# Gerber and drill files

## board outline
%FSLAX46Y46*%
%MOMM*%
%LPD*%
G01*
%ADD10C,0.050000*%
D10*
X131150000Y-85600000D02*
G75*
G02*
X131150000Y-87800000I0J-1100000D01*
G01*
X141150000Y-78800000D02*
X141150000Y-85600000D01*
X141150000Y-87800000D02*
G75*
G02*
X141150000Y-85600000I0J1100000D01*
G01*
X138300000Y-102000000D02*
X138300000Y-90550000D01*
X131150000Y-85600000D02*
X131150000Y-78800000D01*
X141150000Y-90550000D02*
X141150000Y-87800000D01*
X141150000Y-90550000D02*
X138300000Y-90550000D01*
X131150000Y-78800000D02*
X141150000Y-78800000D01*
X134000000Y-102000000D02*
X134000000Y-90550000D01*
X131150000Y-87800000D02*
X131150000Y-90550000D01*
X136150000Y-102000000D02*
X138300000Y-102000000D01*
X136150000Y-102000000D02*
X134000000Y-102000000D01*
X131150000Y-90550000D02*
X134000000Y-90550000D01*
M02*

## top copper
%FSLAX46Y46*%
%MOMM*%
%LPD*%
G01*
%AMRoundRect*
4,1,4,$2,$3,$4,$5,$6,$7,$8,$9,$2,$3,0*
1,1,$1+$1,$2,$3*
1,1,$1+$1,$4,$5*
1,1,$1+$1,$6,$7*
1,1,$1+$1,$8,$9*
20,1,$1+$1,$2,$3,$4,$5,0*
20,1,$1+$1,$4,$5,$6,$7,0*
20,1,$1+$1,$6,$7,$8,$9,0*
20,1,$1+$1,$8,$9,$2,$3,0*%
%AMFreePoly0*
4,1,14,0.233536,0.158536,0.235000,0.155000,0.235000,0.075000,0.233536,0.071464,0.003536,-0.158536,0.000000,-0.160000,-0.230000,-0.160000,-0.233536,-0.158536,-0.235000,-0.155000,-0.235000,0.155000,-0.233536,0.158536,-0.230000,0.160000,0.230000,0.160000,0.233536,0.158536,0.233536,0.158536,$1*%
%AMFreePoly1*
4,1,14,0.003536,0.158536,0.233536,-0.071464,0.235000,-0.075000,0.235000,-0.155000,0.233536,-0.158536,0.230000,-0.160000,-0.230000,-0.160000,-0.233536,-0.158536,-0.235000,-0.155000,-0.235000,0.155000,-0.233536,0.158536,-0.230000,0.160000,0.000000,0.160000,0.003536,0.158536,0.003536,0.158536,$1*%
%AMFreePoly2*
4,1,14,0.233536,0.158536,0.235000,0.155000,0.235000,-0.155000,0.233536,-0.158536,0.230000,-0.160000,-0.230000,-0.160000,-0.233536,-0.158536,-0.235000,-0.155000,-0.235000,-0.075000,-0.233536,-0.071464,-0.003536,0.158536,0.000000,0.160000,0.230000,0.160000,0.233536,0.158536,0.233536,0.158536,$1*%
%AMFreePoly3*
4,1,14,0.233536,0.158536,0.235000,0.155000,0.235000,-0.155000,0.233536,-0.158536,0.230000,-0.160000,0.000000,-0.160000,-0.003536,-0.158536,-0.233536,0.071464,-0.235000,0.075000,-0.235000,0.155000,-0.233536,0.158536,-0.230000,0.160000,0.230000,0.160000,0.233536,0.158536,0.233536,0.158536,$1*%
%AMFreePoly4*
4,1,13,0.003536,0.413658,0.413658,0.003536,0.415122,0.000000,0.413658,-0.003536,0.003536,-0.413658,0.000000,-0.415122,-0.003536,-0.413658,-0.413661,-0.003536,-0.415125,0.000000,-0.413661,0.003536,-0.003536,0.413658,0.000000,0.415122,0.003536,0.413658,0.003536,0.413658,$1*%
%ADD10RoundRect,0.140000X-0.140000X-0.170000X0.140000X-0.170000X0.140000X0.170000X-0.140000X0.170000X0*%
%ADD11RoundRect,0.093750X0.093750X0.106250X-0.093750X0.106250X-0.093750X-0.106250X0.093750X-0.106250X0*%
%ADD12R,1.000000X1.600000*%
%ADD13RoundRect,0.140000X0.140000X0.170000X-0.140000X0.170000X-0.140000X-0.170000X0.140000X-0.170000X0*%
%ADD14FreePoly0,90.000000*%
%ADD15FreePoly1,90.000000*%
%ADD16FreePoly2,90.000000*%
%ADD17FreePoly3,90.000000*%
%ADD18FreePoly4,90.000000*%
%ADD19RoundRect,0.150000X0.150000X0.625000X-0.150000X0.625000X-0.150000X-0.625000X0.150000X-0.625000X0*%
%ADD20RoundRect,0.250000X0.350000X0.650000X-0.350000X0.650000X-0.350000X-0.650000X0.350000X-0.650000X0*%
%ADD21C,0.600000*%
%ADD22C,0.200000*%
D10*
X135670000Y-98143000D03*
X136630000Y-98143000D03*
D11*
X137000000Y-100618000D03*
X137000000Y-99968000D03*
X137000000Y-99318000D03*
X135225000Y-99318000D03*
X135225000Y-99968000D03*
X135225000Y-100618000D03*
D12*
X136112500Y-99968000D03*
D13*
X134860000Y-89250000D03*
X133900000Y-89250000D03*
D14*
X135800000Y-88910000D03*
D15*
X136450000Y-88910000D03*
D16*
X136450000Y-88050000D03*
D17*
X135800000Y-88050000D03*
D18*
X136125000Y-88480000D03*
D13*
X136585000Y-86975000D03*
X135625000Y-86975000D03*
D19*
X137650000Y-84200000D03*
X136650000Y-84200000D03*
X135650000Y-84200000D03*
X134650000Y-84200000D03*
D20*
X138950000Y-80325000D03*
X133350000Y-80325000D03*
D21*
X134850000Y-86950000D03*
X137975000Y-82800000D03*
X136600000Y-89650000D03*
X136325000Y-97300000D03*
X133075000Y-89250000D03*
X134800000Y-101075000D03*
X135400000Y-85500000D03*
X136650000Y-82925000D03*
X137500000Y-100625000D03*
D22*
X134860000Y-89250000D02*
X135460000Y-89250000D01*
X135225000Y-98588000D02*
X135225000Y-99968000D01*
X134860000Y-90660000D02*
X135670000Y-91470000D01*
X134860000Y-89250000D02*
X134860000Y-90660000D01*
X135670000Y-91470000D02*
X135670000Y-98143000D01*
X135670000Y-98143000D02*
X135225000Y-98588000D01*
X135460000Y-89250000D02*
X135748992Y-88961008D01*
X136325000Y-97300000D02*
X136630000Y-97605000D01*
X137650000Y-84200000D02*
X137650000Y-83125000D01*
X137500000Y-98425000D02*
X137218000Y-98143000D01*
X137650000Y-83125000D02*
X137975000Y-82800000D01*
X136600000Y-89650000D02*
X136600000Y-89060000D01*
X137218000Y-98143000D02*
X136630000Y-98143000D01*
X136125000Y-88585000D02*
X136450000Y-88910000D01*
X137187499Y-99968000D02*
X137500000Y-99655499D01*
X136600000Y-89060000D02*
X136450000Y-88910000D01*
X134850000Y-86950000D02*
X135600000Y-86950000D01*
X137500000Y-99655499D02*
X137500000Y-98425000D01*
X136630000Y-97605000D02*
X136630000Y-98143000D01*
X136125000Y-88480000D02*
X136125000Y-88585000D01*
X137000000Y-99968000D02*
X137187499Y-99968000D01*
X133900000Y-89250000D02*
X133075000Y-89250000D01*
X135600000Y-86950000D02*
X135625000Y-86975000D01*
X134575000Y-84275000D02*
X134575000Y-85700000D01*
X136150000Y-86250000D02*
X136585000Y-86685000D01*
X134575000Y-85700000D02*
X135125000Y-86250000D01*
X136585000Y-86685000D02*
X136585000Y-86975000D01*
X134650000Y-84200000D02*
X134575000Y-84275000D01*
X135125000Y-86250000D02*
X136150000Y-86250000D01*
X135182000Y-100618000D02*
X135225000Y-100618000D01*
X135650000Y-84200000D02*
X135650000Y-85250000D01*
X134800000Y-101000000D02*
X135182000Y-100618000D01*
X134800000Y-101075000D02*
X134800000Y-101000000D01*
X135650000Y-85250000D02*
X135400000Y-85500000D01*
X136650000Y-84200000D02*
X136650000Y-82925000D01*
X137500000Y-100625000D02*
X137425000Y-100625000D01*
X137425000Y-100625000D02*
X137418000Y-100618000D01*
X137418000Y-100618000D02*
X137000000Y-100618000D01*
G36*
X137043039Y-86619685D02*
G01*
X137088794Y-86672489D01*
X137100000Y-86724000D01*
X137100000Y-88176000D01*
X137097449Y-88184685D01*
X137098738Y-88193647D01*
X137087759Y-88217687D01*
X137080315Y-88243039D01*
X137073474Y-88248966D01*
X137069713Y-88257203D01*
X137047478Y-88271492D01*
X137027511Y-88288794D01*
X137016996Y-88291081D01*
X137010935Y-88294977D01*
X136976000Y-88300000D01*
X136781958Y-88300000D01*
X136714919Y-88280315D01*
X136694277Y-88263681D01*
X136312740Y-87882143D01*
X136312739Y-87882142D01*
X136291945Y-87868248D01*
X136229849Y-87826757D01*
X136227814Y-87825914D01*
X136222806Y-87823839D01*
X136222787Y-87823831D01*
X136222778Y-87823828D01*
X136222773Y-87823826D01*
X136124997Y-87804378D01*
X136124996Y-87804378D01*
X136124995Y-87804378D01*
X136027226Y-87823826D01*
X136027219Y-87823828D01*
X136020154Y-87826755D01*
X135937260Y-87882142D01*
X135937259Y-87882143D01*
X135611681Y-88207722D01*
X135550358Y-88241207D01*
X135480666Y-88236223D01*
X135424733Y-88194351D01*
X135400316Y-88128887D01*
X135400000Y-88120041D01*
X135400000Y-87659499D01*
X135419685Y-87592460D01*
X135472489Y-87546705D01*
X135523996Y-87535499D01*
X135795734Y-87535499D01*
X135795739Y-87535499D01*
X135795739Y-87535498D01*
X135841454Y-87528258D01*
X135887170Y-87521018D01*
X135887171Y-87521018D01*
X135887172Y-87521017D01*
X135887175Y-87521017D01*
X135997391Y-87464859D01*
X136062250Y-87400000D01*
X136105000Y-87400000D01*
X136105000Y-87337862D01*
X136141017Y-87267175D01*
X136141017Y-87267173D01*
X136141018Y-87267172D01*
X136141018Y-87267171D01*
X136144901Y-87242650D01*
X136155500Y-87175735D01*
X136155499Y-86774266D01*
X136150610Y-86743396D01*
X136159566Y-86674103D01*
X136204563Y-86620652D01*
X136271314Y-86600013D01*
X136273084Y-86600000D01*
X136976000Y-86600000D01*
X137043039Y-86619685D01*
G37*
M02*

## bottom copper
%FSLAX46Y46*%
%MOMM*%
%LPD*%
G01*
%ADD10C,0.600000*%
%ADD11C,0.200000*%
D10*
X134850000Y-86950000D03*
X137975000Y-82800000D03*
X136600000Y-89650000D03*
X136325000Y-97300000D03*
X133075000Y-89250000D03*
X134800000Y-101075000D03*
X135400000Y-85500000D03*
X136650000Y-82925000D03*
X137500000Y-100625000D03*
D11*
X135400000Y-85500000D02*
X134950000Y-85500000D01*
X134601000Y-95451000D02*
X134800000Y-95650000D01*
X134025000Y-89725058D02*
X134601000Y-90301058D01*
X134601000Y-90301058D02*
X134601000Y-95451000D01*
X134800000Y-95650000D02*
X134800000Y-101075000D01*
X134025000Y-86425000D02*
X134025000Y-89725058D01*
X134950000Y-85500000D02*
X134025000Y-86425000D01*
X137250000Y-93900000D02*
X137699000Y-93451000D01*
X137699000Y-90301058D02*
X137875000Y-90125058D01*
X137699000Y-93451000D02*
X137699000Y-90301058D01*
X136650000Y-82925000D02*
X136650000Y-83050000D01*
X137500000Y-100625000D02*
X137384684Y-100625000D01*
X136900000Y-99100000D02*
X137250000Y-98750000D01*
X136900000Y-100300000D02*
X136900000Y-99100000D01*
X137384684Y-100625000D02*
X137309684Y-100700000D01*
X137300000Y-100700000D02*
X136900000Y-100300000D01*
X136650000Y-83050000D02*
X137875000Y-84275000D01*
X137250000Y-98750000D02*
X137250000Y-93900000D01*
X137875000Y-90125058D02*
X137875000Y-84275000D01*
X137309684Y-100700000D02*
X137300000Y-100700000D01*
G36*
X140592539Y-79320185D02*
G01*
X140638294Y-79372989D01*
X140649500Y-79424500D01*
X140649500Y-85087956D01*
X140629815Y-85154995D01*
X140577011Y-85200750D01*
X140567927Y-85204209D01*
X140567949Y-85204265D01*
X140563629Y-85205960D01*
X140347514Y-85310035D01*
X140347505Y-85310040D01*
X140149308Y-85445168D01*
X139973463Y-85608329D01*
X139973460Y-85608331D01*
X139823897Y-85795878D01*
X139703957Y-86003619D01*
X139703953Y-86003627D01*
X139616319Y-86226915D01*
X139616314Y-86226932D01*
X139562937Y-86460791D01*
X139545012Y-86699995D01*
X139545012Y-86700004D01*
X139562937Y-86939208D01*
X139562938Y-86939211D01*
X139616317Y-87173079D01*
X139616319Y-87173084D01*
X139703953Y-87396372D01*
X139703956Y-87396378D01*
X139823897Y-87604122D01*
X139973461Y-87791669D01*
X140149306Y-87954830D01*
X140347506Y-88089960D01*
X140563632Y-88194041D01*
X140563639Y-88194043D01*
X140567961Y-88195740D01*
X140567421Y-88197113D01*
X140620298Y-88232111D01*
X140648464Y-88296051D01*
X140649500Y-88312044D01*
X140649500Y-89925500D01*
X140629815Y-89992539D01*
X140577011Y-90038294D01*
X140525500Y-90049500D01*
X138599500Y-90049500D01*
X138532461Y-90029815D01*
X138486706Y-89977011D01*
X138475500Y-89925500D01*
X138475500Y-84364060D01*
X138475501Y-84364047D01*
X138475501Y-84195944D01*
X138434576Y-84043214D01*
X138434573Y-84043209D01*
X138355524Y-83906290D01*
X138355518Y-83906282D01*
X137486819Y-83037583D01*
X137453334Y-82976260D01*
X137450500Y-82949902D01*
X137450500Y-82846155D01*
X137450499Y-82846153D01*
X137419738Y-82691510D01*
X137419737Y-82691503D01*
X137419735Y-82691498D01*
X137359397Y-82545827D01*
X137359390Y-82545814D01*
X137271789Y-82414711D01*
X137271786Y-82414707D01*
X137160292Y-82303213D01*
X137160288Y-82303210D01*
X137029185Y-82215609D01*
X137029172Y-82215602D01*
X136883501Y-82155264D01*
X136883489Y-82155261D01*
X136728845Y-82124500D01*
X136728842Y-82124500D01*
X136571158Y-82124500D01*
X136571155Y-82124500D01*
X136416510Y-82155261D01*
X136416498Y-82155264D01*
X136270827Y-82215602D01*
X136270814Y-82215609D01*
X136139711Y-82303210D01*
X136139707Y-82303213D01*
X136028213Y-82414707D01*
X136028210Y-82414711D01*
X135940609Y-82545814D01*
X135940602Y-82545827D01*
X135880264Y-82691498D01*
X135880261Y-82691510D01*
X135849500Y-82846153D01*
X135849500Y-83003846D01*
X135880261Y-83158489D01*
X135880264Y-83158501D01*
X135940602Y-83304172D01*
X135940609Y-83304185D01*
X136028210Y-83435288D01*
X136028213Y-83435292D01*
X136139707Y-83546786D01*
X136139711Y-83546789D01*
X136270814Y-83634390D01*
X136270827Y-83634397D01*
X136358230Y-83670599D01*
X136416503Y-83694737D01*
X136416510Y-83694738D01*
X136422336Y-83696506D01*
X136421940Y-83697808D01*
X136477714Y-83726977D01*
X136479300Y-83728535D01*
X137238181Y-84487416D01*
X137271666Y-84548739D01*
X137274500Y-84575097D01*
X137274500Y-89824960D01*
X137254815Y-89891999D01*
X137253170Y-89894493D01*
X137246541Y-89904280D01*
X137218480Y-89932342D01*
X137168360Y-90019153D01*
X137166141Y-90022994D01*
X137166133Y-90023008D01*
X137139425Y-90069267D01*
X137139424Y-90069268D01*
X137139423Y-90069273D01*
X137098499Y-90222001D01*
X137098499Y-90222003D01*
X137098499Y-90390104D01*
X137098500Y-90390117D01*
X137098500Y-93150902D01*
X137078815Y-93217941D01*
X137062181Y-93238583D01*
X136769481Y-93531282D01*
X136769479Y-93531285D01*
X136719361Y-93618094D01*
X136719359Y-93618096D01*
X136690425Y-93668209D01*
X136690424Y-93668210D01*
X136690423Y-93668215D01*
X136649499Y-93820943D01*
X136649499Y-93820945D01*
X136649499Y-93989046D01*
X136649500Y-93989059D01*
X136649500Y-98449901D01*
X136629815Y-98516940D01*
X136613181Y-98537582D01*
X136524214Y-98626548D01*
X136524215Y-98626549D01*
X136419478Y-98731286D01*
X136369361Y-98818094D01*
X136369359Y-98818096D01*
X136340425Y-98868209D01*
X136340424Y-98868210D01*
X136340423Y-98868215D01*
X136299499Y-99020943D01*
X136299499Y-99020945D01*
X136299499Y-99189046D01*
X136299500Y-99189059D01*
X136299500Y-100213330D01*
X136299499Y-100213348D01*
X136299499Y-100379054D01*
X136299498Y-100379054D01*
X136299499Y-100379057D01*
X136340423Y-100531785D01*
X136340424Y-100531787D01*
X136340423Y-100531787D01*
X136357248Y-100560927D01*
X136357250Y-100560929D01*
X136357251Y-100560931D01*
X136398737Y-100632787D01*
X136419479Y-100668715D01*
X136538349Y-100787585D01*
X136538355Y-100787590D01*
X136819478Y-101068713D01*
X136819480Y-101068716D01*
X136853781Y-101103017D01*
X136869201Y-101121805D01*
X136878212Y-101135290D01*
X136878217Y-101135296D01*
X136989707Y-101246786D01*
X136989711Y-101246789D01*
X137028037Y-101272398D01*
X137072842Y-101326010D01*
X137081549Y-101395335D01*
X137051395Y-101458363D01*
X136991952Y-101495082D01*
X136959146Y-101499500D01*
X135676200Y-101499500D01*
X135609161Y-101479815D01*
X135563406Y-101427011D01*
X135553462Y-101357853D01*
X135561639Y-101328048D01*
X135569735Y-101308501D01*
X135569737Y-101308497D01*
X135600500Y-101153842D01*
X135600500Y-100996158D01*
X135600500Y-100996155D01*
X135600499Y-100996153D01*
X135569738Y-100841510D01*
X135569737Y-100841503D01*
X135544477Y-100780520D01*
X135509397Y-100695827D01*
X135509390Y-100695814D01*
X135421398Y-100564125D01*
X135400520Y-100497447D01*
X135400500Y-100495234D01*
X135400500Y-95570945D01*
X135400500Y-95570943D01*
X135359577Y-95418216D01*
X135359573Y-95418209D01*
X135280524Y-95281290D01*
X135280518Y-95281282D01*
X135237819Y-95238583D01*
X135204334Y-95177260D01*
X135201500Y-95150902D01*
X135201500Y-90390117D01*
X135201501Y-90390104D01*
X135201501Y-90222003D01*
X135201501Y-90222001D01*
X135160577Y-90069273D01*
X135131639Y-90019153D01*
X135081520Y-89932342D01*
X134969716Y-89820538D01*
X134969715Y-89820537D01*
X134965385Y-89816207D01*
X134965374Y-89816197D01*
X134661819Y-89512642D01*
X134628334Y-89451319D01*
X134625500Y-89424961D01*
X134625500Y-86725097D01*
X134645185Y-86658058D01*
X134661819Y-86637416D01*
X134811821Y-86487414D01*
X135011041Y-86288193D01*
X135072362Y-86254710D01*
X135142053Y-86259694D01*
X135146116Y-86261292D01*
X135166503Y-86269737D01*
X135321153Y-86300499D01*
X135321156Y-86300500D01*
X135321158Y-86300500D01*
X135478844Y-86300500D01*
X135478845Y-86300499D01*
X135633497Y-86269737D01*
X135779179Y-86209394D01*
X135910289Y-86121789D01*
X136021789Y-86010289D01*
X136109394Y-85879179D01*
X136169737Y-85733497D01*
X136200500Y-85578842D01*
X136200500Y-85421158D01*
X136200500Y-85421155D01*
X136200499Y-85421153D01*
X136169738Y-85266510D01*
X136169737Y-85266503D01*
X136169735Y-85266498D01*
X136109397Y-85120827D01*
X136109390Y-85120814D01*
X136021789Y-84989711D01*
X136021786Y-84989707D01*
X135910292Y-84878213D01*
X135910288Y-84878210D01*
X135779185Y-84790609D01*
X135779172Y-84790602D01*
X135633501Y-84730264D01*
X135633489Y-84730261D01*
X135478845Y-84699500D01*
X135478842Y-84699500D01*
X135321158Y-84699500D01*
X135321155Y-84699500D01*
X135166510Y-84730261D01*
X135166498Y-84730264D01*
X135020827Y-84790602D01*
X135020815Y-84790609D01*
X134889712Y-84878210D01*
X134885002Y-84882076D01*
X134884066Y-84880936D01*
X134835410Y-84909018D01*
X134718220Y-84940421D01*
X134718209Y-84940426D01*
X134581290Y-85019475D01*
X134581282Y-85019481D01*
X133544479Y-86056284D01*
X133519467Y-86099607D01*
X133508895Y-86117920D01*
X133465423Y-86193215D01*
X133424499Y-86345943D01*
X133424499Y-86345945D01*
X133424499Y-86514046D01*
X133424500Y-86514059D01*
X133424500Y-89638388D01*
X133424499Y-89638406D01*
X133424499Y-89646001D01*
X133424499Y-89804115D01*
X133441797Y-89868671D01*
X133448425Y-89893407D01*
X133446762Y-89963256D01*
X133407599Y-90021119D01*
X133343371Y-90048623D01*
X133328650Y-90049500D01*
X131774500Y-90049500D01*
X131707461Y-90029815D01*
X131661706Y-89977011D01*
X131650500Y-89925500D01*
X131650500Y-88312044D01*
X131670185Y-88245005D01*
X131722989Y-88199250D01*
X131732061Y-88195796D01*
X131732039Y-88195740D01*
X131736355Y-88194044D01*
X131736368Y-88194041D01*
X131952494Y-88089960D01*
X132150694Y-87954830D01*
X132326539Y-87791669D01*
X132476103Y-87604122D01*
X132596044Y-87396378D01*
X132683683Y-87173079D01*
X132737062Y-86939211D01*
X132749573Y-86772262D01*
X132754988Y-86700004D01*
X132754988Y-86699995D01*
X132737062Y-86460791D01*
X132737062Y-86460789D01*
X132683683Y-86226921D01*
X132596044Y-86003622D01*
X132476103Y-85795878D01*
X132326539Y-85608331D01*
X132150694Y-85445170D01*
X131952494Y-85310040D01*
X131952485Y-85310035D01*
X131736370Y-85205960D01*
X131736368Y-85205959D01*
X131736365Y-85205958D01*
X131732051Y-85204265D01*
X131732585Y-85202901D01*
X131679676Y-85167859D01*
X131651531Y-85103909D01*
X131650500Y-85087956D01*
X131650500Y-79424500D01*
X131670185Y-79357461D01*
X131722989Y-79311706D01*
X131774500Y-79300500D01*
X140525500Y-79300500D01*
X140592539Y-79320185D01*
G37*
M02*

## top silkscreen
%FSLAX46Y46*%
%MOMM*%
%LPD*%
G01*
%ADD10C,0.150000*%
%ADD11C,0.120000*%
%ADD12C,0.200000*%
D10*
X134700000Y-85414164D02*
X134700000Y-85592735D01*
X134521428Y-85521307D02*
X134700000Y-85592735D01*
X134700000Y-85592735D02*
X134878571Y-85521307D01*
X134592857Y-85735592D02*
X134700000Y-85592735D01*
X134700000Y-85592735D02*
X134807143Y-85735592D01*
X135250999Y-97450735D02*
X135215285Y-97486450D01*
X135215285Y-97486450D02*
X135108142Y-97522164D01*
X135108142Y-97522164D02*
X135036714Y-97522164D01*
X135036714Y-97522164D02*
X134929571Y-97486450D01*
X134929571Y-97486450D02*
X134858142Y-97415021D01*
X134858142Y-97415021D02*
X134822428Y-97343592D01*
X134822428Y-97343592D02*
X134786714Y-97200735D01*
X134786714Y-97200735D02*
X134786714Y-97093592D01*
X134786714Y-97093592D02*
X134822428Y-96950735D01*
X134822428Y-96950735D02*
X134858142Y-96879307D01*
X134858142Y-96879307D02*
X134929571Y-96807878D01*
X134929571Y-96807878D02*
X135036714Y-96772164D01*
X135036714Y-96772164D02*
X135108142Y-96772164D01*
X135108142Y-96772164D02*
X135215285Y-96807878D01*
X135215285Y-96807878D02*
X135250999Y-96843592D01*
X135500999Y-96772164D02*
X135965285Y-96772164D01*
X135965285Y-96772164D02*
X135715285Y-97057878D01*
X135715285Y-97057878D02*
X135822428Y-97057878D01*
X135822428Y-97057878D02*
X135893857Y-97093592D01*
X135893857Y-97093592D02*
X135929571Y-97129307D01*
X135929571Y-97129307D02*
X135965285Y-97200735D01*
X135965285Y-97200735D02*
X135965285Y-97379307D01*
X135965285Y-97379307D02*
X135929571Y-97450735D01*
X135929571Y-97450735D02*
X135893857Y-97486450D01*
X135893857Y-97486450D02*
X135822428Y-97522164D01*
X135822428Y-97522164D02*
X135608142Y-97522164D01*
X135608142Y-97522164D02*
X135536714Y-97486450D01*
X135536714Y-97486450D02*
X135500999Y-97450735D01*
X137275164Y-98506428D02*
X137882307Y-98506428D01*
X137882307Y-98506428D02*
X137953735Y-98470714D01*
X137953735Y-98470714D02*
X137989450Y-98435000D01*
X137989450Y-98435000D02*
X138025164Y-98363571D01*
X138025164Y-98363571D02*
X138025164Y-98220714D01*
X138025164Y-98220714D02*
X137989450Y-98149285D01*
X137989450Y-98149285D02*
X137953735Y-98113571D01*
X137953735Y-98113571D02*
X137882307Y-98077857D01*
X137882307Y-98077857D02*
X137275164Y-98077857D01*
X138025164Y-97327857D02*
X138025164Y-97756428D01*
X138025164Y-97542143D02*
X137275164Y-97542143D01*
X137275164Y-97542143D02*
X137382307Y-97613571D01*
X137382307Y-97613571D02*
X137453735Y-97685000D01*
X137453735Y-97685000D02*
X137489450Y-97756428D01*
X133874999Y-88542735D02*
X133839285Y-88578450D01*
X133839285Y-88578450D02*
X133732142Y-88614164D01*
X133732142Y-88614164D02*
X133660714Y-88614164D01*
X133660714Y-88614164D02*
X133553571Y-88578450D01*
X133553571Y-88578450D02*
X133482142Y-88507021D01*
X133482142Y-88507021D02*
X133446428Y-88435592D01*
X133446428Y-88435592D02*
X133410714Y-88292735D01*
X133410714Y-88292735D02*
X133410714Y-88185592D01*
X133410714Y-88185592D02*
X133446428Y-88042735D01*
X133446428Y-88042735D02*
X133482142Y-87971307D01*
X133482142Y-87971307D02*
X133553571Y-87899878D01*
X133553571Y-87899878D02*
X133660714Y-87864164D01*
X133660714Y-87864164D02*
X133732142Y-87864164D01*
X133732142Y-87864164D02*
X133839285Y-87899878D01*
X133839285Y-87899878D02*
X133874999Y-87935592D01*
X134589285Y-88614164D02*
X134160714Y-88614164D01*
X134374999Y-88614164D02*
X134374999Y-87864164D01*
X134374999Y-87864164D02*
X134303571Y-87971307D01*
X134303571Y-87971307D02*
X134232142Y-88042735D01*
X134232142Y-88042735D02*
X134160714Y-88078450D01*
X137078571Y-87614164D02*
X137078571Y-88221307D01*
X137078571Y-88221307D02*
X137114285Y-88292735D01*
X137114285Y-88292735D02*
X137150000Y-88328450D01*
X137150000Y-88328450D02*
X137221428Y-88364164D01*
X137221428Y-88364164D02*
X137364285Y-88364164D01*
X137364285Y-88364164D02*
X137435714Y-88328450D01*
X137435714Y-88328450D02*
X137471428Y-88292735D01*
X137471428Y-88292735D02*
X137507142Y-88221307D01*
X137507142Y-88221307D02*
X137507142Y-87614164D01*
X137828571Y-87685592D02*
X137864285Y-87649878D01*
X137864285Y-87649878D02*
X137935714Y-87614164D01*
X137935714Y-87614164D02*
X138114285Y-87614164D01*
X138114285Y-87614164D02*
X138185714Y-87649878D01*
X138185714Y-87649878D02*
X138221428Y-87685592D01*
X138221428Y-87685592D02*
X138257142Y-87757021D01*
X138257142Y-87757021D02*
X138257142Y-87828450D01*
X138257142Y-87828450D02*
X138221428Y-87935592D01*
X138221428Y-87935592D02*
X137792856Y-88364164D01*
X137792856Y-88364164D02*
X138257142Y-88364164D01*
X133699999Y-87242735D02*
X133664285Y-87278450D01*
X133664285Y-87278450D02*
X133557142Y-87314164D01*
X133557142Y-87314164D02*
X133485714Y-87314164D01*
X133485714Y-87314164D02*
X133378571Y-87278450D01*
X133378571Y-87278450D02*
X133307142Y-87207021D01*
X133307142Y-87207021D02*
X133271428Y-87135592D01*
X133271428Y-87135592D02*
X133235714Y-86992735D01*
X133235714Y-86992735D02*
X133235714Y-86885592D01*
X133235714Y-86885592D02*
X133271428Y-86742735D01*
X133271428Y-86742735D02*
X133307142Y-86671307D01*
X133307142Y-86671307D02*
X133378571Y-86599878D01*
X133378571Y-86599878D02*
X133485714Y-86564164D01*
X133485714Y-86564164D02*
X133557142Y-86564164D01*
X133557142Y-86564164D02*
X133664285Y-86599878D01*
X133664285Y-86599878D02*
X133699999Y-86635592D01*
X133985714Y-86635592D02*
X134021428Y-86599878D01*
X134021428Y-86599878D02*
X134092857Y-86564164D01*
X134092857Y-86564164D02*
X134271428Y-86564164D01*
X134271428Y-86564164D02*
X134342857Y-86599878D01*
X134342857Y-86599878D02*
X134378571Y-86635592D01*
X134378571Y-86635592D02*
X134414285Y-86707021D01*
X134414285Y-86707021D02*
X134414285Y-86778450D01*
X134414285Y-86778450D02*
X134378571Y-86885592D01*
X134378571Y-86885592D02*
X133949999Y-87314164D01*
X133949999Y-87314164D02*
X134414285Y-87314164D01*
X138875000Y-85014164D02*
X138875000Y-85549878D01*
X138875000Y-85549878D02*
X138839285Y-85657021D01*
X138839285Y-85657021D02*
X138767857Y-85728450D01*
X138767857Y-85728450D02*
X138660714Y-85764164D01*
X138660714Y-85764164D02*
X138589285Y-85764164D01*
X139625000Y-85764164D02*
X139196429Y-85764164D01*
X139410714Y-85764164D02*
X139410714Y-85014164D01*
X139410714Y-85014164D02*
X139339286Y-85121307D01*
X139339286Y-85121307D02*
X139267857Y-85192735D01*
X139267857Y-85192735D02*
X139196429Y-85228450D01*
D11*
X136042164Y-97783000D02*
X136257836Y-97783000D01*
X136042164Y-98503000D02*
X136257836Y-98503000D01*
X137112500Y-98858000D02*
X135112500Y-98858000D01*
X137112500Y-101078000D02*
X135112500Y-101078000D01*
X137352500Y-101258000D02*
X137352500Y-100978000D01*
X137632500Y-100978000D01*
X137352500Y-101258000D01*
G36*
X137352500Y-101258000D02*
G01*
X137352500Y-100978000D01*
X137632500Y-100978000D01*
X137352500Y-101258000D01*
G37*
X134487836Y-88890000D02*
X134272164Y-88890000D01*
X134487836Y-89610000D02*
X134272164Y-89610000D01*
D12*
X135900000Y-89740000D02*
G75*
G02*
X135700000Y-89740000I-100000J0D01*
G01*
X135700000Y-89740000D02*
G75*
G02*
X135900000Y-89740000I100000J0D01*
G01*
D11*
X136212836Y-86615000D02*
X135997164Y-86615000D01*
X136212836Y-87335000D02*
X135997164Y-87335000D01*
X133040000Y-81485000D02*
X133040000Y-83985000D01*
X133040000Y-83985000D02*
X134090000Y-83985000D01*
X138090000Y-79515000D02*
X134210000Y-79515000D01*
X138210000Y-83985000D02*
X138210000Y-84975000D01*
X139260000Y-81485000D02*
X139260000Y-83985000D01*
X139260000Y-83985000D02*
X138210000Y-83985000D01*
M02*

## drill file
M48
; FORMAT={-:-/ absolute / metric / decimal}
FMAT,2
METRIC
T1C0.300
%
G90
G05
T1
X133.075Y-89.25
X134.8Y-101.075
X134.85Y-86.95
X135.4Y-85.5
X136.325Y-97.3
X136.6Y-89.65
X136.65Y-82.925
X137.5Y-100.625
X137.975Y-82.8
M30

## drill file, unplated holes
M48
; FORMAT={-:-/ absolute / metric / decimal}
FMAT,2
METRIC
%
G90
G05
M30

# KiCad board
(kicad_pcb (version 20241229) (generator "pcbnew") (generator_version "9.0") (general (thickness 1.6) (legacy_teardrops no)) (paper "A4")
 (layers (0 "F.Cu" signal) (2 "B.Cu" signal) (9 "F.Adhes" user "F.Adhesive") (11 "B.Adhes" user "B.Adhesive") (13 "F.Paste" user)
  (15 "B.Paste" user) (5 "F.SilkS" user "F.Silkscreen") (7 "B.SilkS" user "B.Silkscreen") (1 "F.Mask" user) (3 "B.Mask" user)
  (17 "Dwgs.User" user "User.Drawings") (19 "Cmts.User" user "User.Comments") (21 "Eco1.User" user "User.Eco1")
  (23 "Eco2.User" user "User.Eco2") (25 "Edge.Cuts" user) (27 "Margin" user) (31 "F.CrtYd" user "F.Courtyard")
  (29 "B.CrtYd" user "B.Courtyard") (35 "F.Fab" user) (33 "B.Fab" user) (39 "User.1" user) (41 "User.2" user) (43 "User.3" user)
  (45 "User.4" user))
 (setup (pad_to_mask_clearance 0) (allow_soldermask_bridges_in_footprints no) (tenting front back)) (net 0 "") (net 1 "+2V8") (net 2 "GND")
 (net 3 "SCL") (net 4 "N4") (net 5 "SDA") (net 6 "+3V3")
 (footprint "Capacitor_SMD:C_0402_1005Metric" (layer "F.Cu") (at 136.15 98.143)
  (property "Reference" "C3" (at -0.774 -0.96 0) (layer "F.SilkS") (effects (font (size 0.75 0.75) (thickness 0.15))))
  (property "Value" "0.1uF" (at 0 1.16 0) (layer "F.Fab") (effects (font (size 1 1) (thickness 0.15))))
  (fp_line (start -0.107836 -0.36) (end 0.107836 -0.36) (stroke (width 0.12) (type solid)) (layer "F.SilkS"))
  (fp_line (start -0.107836 0.36) (end 0.107836 0.36) (stroke (width 0.12) (type solid)) (layer "F.SilkS"))
  (pad "1" smd roundrect (at -0.48 0) (size 0.56 0.62) (layers "F.Cu" "F.Mask" "F.Paste") (roundrect_rratio 0.25) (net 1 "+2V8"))
  (pad "2" smd roundrect (at 0.48 0) (size 0.56 0.62) (layers "F.Cu" "F.Mask" "F.Paste") (roundrect_rratio 0.25) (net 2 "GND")))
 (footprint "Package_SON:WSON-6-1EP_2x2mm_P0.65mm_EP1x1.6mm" (layer "F.Cu") (at 136.1125 99.968 180)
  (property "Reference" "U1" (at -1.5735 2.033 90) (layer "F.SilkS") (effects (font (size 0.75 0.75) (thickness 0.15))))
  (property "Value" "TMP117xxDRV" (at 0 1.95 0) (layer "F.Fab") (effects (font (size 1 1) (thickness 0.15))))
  (fp_line (start -1 1.11) (end 1 1.11) (stroke (width 0.12) (type solid)) (layer "F.SilkS"))
  (fp_line (start -1 -1.11) (end 1 -1.11) (stroke (width 0.12) (type solid)) (layer "F.SilkS"))
  (fp_poly (pts (xy -1.24 -1.01) (xy -1.52 -1.01) (xy -1.24 -1.29)) (stroke (width 0.12) (type solid)) (fill yes) (layer "F.SilkS"))
  (pad "" smd roundrect (at 0 -0.4 180) (size 0.81 0.64) (layers "F.Paste") (roundrect_rratio 0.25))
  (pad "" smd roundrect (at 0 0.4 180) (size 0.81 0.64) (layers "F.Paste") (roundrect_rratio 0.25))
  (pad "1" smd roundrect (at -0.8875 -0.65 180) (size 0.375 0.4) (layers "F.Cu" "F.Mask" "F.Paste") (roundrect_rratio 0.25) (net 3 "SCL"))
  (pad "2" smd roundrect (at -0.8875 0 180) (size 0.375 0.4) (layers "F.Cu" "F.Mask" "F.Paste") (roundrect_rratio 0.25) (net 2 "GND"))
  (pad "3" smd roundrect (at -0.8875 0.65 180) (size 0.375 0.4) (layers "F.Cu" "F.Mask" "F.Paste") (roundrect_rratio 0.25) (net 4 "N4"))
  (pad "4" smd roundrect (at 0.8875 0.65 180) (size 0.375 0.4) (layers "F.Cu" "F.Mask" "F.Paste") (roundrect_rratio 0.25) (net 1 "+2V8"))
  (pad "5" smd roundrect (at 0.8875 0 180) (size 0.375 0.4) (layers "F.Cu" "F.Mask" "F.Paste") (roundrect_rratio 0.25) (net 1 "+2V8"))
  (pad "6" smd roundrect (at 0.8875 -0.65 180) (size 0.375 0.4) (layers "F.Cu" "F.Mask" "F.Paste") (roundrect_rratio 0.25) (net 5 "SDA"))
  (pad "7" smd rect (at 0 0 180) (size 1 1.6) (layers "F.Cu" "F.Mask") (zone_connect 2)))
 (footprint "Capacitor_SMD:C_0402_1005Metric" (layer "F.Cu") (at 134.38 89.25 180)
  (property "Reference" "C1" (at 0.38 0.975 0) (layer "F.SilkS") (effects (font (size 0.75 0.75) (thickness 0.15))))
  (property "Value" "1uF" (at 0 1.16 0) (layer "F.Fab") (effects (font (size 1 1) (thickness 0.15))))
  (fp_line (start -0.107836 0.36) (end 0.107836 0.36) (stroke (width 0.12) (type solid)) (layer "F.SilkS"))
  (fp_line (start -0.107836 -0.36) (end 0.107836 -0.36) (stroke (width 0.12) (type solid)) (layer "F.SilkS"))
  (pad "1" smd roundrect (at -0.48 0 180) (size 0.56 0.62) (layers "F.Cu" "F.Mask" "F.Paste") (roundrect_rratio 0.25) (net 1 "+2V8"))
  (pad "2" smd roundrect (at 0.48 0 180) (size 0.56 0.62) (layers "F.Cu" "F.Mask" "F.Paste") (roundrect_rratio 0.25) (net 2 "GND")))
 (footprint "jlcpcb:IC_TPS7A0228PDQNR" (layer "F.Cu") (at 136.125 88.48 90)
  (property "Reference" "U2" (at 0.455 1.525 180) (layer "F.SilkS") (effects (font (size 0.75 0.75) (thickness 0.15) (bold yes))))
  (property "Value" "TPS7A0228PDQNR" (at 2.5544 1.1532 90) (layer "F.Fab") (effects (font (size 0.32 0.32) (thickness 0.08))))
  (fp_circle (center -1.26 -0.325) (end -1.16 -0.325) (stroke (width 0.2) (type solid)) (fill no) (layer "F.SilkS"))
  (pad "1" smd custom (at -0.43 -0.325 90) (size 0.05 0.05) (layers "F.Cu") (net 1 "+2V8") (options (clearance outline) (anchor rect))
   (primitives))
  (pad "2" smd custom (at -0.43 0.325 90) (size 0.05 0.05) (layers "F.Cu") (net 2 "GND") (options (clearance outline) (anchor rect))
   (primitives))
  (pad "3" smd custom (at 0.43 0.325 90) (size 0.05 0.05) (layers "F.Cu") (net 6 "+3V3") (options (clearance outline) (anchor rect))
   (primitives))
  (pad "4" smd custom (at 0.43 -0.325 90) (size 0.05 0.05) (layers "F.Cu") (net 6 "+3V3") (options (clearance outline) (anchor rect))
   (primitives))
  (pad "5" smd custom (at 0 0 90) (size 0.05 0.05) (layers "F.Cu") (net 2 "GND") (options (clearance outline) (anchor rect)) (primitives)))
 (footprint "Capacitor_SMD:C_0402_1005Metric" (layer "F.Cu") (at 136.105 86.975 180)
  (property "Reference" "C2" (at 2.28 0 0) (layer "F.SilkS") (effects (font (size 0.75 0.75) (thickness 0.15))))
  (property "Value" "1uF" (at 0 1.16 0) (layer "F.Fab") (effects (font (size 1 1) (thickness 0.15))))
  (fp_line (start -0.107836 0.36) (end 0.107836 0.36) (stroke (width 0.12) (type solid)) (layer "F.SilkS"))
  (fp_line (start -0.107836 -0.36) (end 0.107836 -0.36) (stroke (width 0.12) (type solid)) (layer "F.SilkS"))
  (pad "1" smd roundrect (at -0.48 0 180) (size 0.56 0.62) (layers "F.Cu" "F.Mask" "F.Paste") (roundrect_rratio 0.25) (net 6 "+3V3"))
  (pad "2" smd roundrect (at 0.48 0 180) (size 0.56 0.62) (layers "F.Cu" "F.Mask" "F.Paste") (roundrect_rratio 0.25) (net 2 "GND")))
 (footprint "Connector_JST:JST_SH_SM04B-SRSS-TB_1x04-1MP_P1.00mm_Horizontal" (layer "F.Cu") (at 136.15 82.2 180)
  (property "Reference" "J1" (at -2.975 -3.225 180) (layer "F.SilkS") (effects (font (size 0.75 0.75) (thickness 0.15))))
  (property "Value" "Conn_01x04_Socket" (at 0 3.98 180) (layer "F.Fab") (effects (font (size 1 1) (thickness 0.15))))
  (fp_line (start 3.11 0.715) (end 3.11 -1.785) (stroke (width 0.12) (type solid)) (layer "F.SilkS"))
  (fp_line (start 3.11 -1.785) (end 2.06 -1.785) (stroke (width 0.12) (type solid)) (layer "F.SilkS"))
  (fp_line (start -1.94 2.685) (end 1.94 2.685) (stroke (width 0.12) (type solid)) (layer "F.SilkS"))
  (fp_line (start -2.06 -1.785) (end -2.06 -2.775) (stroke (width 0.12) (type solid)) (layer "F.SilkS"))
  (fp_line (start -3.11 0.715) (end -3.11 -1.785) (stroke (width 0.12) (type solid)) (layer "F.SilkS"))
  (fp_line (start -3.11 -1.785) (end -2.06 -1.785) (stroke (width 0.12) (type solid)) (layer "F.SilkS"))
  (pad "1" smd roundrect (at -1.5 -2 180) (size 0.6 1.55) (layers "F.Cu" "F.Mask" "F.Paste") (roundrect_rratio 0.25) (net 2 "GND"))
  (pad "2" smd roundrect (at -0.5 -2 180) (size 0.6 1.55) (layers "F.Cu" "F.Mask" "F.Paste") (roundrect_rratio 0.25) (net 3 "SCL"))
  (pad "3" smd roundrect (at 0.5 -2 180) (size 0.6 1.55) (layers "F.Cu" "F.Mask" "F.Paste") (roundrect_rratio 0.25) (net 5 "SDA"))
  (pad "4" smd roundrect (at 1.5 -2 180) (size 0.6 1.55) (layers "F.Cu" "F.Mask" "F.Paste") (roundrect_rratio 0.25) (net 6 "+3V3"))
  (pad "MP" smd roundrect (at -2.8 1.875 180) (size 1.2 1.8) (layers "F.Cu" "F.Mask" "F.Paste") (roundrect_rratio 0.208333))
  (pad "MP" smd roundrect (at 2.8 1.875 180) (size 1.2 1.8) (layers "F.Cu" "F.Mask" "F.Paste") (roundrect_rratio 0.208333)))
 (gr_arc (start 131.15 85.6) (mid 132.25 86.7) (end 131.15 87.8) (stroke (width 0.05) (type default)) (layer "Edge.Cuts"))
 (gr_line (start 141.15 78.8) (end 141.15 85.6) (stroke (width 0.05) (type solid)) (layer "Edge.Cuts"))
 (gr_arc (start 141.15 87.8) (mid 140.05 86.7) (end 141.15 85.6) (stroke (width 0.05) (type solid)) (layer "Edge.Cuts"))
 (gr_line (start 138.3 102) (end 138.3 90.55) (stroke (width 0.05) (type default)) (layer "Edge.Cuts"))
 (gr_line (start 131.15 85.6) (end 131.15 78.8) (stroke (width 0.05) (type solid)) (layer "Edge.Cuts"))
 (gr_line (start 141.15 90.55) (end 141.15 87.8) (stroke (width 0.05) (type default)) (layer "Edge.Cuts"))
 (gr_line (start 141.15 90.55) (end 138.3 90.55) (stroke (width 0.05) (type solid)) (layer "Edge.Cuts"))
 (gr_line (start 131.15 78.8) (end 141.15 78.8) (stroke (width 0.05) (type solid)) (layer "Edge.Cuts"))
 (gr_line (start 134 102) (end 134 90.55) (stroke (width 0.05) (type default)) (layer "Edge.Cuts"))
 (gr_line (start 131.15 87.8) (end 131.15 90.55) (stroke (width 0.05) (type default)) (layer "Edge.Cuts"))
 (gr_line (start 136.15 102) (end 138.3 102) (stroke (width 0.05) (type solid)) (layer "Edge.Cuts"))
 (gr_line (start 136.15 102) (end 134 102) (stroke (width 0.05) (type solid)) (layer "Edge.Cuts"))
 (gr_line (start 131.15 90.55) (end 134 90.55) (stroke (width 0.05) (type solid)) (layer "Edge.Cuts"))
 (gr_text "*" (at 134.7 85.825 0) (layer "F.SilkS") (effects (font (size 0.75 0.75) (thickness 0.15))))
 (segment (start 134.86 89.25) (end 135.46 89.25) (width 0.2) (layer "F.Cu") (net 1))
 (segment (start 135.225 98.588) (end 135.225 99.968) (width 0.2) (layer "F.Cu") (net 1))
 (segment (start 134.86 90.66) (end 135.67 91.47) (width 0.2) (layer "F.Cu") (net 1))
 (segment (start 134.86 89.25) (end 134.86 90.66) (width 0.2) (layer "F.Cu") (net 1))
 (segment (start 135.67 91.47) (end 135.67 98.143) (width 0.2) (layer "F.Cu") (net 1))
 (segment (start 135.67 98.143) (end 135.225 98.588) (width 0.2) (layer "F.Cu") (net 1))
 (segment (start 135.46 89.25) (end 135.748992 88.961008) (width 0.2) (layer "F.Cu") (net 1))
 (segment (start 136.325 97.3) (end 136.63 97.605) (width 0.2) (layer "F.Cu") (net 2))
 (segment (start 137.65 84.2) (end 137.65 83.125) (width 0.2) (layer "F.Cu") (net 2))
 (segment (start 137.5 98.425) (end 137.218 98.143) (width 0.2) (layer "F.Cu") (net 2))
 (segment (start 137.65 83.125) (end 137.975 82.8) (width 0.2) (layer "F.Cu") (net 2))
 (segment (start 136.6 89.65) (end 136.6 89.06) (width 0.2) (layer "F.Cu") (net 2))
 (segment (start 137.218 98.143) (end 136.63 98.143) (width 0.2) (layer "F.Cu") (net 2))
 (segment (start 136.125 88.585) (end 136.45 88.91) (width 0.2) (layer "F.Cu") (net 2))
 (segment (start 137.187499 99.968) (end 137.5 99.655499) (width 0.2) (layer "F.Cu") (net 2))
 (segment (start 136.6 89.06) (end 136.45 88.91) (width 0.2) (layer "F.Cu") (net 2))
 (segment (start 134.85 86.95) (end 135.6 86.95) (width 0.2) (layer "F.Cu") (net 2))
 (segment (start 137.5 99.655499) (end 137.5 98.425) (width 0.2) (layer "F.Cu") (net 2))
 (segment (start 136.63 97.605) (end 136.63 98.143) (width 0.2) (layer "F.Cu") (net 2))
 (segment (start 136.125 88.48) (end 136.125 88.585) (width 0.2) (layer "F.Cu") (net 2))
 (segment (start 137 99.968) (end 137.187499 99.968) (width 0.2) (layer "F.Cu") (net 2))
 (segment (start 133.9 89.25) (end 133.075 89.25) (width 0.2) (layer "F.Cu") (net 2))
 (segment (start 135.6 86.95) (end 135.625 86.975) (width 0.2) (layer "F.Cu") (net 2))
 (via (at 134.85 86.95) (size 0.6) (drill 0.3) (layers "F.Cu" "B.Cu") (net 2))
 (via (at 137.975 82.8) (size 0.6) (drill 0.3) (layers "F.Cu" "B.Cu") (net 2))
 (via (at 136.6 89.65) (size 0.6) (drill 0.3) (layers "F.Cu" "B.Cu") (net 2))
 (via (at 136.325 97.3) (size 0.6) (drill 0.3) (layers "F.Cu" "B.Cu") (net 2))
 (via (at 133.075 89.25) (size 0.6) (drill 0.3) (layers "F.Cu" "B.Cu") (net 2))
 (segment (start 134.575 84.275) (end 134.575 85.7) (width 0.2) (layer "F.Cu") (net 6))
 (segment (start 136.15 86.25) (end 136.585 86.685) (width 0.2) (layer "F.Cu") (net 6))
 (segment (start 134.575 85.7) (end 135.125 86.25) (width 0.2) (layer "F.Cu") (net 6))
 (segment (start 136.585 86.685) (end 136.585 86.975) (width 0.2) (layer "F.Cu") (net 6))
 (segment (start 134.65 84.2) (end 134.575 84.275) (width 0.2) (layer "F.Cu") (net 6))
 (segment (start 135.125 86.25) (end 136.15 86.25) (width 0.2) (layer "F.Cu") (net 6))
 (segment (start 135.182 100.618) (end 135.225 100.618) (width 0.2) (layer "F.Cu") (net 5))
 (segment (start 135.65 84.2) (end 135.65 85.25) (width 0.2) (layer "F.Cu") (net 5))
 (segment (start 134.8 101) (end 135.182 100.618) (width 0.2) (layer "F.Cu") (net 5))
 (segment (start 134.8 101.075) (end 134.8 101) (width 0.2) (layer "F.Cu") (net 5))
 (segment (start 135.65 85.25) (end 135.4 85.5) (width 0.2) (layer "F.Cu") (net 5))
 (via (at 134.8 101.075) (size 0.6) (drill 0.3) (layers "F.Cu" "B.Cu") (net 5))
 (via (at 135.4 85.5) (size 0.6) (drill 0.3) (layers "F.Cu" "B.Cu") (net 5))
 (segment (start 135.4 85.5) (end 134.95 85.5) (width 0.2) (layer "B.Cu") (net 5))
 (segment (start 134.601 95.451) (end 134.8 95.65) (width 0.2) (layer "B.Cu") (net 5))
 (segment (start 134.025 89.725058) (end 134.601 90.301058) (width 0.2) (layer "B.Cu") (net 5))
 (segment (start 134.601 90.301058) (end 134.601 95.451) (width 0.2) (layer "B.Cu") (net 5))
 (segment (start 134.8 95.65) (end 134.8 101.075) (width 0.2) (layer "B.Cu") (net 5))
 (segment (start 134.025 86.425) (end 134.025 89.725058) (width 0.2) (layer "B.Cu") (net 5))
 (segment (start 134.95 85.5) (end 134.025 86.425) (width 0.2) (layer "B.Cu") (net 5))
 (segment (start 136.65 84.2) (end 136.65 82.925) (width 0.2) (layer "F.Cu") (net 3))
 (segment (start 137.5 100.625) (end 137.425 100.625) (width 0.2) (layer "F.Cu") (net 3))
 (segment (start 137.425 100.625) (end 137.418 100.618) (width 0.2) (layer "F.Cu") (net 3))
 (segment (start 137.418 100.618) (end 137 100.618) (width 0.2) (layer "F.Cu") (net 3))
 (via (at 136.65 82.925) (size 0.6) (drill 0.3) (layers "F.Cu" "B.Cu") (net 3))
 (via (at 137.5 100.625) (size 0.6) (drill 0.3) (layers "F.Cu" "B.Cu") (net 3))
 (segment (start 137.25 93.9) (end 137.699 93.451) (width 0.2) (layer "B.Cu") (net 3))
 (segment (start 137.699 90.301058) (end 137.875 90.125058) (width 0.2) (layer "B.Cu") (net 3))
 (segment (start 137.699 93.451) (end 137.699 90.301058) (width 0.2) (layer "B.Cu") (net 3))
 (segment (start 136.65 82.925) (end 136.65 83.05) (width 0.2) (layer "B.Cu") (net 3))
 (segment (start 137.5 100.625) (end 137.384684 100.625) (width 0.2) (layer "B.Cu") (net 3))
 (segment (start 136.9 99.1) (end 137.25 98.75) (width 0.2) (layer "B.Cu") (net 3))
 (segment (start 136.9 100.3) (end 136.9 99.1) (width 0.2) (layer "B.Cu") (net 3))
 (segment (start 137.384684 100.625) (end 137.309684 100.7) (width 0.2) (layer "B.Cu") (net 3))
 (segment (start 137.3 100.7) (end 136.9 100.3) (width 0.2) (layer "B.Cu") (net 3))
 (segment (start 136.65 83.05) (end 137.875 84.275) (width 0.2) (layer "B.Cu") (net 3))
 (segment (start 137.25 98.75) (end 137.25 93.9) (width 0.2) (layer "B.Cu") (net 3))
 (segment (start 137.875 90.125058) (end 137.875 84.275) (width 0.2) (layer "B.Cu") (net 3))
 (segment (start 137.309684 100.7) (end 137.3 100.7) (width 0.2) (layer "B.Cu") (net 3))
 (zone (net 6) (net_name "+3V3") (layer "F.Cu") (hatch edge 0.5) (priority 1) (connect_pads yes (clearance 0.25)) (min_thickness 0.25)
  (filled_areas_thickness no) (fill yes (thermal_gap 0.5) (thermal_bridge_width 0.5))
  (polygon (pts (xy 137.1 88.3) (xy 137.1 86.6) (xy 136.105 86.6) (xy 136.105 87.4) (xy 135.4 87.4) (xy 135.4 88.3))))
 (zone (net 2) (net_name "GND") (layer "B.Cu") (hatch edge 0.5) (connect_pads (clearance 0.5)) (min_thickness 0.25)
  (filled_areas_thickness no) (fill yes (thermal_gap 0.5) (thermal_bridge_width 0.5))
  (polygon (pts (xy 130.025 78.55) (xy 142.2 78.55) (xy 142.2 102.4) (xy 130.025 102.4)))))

